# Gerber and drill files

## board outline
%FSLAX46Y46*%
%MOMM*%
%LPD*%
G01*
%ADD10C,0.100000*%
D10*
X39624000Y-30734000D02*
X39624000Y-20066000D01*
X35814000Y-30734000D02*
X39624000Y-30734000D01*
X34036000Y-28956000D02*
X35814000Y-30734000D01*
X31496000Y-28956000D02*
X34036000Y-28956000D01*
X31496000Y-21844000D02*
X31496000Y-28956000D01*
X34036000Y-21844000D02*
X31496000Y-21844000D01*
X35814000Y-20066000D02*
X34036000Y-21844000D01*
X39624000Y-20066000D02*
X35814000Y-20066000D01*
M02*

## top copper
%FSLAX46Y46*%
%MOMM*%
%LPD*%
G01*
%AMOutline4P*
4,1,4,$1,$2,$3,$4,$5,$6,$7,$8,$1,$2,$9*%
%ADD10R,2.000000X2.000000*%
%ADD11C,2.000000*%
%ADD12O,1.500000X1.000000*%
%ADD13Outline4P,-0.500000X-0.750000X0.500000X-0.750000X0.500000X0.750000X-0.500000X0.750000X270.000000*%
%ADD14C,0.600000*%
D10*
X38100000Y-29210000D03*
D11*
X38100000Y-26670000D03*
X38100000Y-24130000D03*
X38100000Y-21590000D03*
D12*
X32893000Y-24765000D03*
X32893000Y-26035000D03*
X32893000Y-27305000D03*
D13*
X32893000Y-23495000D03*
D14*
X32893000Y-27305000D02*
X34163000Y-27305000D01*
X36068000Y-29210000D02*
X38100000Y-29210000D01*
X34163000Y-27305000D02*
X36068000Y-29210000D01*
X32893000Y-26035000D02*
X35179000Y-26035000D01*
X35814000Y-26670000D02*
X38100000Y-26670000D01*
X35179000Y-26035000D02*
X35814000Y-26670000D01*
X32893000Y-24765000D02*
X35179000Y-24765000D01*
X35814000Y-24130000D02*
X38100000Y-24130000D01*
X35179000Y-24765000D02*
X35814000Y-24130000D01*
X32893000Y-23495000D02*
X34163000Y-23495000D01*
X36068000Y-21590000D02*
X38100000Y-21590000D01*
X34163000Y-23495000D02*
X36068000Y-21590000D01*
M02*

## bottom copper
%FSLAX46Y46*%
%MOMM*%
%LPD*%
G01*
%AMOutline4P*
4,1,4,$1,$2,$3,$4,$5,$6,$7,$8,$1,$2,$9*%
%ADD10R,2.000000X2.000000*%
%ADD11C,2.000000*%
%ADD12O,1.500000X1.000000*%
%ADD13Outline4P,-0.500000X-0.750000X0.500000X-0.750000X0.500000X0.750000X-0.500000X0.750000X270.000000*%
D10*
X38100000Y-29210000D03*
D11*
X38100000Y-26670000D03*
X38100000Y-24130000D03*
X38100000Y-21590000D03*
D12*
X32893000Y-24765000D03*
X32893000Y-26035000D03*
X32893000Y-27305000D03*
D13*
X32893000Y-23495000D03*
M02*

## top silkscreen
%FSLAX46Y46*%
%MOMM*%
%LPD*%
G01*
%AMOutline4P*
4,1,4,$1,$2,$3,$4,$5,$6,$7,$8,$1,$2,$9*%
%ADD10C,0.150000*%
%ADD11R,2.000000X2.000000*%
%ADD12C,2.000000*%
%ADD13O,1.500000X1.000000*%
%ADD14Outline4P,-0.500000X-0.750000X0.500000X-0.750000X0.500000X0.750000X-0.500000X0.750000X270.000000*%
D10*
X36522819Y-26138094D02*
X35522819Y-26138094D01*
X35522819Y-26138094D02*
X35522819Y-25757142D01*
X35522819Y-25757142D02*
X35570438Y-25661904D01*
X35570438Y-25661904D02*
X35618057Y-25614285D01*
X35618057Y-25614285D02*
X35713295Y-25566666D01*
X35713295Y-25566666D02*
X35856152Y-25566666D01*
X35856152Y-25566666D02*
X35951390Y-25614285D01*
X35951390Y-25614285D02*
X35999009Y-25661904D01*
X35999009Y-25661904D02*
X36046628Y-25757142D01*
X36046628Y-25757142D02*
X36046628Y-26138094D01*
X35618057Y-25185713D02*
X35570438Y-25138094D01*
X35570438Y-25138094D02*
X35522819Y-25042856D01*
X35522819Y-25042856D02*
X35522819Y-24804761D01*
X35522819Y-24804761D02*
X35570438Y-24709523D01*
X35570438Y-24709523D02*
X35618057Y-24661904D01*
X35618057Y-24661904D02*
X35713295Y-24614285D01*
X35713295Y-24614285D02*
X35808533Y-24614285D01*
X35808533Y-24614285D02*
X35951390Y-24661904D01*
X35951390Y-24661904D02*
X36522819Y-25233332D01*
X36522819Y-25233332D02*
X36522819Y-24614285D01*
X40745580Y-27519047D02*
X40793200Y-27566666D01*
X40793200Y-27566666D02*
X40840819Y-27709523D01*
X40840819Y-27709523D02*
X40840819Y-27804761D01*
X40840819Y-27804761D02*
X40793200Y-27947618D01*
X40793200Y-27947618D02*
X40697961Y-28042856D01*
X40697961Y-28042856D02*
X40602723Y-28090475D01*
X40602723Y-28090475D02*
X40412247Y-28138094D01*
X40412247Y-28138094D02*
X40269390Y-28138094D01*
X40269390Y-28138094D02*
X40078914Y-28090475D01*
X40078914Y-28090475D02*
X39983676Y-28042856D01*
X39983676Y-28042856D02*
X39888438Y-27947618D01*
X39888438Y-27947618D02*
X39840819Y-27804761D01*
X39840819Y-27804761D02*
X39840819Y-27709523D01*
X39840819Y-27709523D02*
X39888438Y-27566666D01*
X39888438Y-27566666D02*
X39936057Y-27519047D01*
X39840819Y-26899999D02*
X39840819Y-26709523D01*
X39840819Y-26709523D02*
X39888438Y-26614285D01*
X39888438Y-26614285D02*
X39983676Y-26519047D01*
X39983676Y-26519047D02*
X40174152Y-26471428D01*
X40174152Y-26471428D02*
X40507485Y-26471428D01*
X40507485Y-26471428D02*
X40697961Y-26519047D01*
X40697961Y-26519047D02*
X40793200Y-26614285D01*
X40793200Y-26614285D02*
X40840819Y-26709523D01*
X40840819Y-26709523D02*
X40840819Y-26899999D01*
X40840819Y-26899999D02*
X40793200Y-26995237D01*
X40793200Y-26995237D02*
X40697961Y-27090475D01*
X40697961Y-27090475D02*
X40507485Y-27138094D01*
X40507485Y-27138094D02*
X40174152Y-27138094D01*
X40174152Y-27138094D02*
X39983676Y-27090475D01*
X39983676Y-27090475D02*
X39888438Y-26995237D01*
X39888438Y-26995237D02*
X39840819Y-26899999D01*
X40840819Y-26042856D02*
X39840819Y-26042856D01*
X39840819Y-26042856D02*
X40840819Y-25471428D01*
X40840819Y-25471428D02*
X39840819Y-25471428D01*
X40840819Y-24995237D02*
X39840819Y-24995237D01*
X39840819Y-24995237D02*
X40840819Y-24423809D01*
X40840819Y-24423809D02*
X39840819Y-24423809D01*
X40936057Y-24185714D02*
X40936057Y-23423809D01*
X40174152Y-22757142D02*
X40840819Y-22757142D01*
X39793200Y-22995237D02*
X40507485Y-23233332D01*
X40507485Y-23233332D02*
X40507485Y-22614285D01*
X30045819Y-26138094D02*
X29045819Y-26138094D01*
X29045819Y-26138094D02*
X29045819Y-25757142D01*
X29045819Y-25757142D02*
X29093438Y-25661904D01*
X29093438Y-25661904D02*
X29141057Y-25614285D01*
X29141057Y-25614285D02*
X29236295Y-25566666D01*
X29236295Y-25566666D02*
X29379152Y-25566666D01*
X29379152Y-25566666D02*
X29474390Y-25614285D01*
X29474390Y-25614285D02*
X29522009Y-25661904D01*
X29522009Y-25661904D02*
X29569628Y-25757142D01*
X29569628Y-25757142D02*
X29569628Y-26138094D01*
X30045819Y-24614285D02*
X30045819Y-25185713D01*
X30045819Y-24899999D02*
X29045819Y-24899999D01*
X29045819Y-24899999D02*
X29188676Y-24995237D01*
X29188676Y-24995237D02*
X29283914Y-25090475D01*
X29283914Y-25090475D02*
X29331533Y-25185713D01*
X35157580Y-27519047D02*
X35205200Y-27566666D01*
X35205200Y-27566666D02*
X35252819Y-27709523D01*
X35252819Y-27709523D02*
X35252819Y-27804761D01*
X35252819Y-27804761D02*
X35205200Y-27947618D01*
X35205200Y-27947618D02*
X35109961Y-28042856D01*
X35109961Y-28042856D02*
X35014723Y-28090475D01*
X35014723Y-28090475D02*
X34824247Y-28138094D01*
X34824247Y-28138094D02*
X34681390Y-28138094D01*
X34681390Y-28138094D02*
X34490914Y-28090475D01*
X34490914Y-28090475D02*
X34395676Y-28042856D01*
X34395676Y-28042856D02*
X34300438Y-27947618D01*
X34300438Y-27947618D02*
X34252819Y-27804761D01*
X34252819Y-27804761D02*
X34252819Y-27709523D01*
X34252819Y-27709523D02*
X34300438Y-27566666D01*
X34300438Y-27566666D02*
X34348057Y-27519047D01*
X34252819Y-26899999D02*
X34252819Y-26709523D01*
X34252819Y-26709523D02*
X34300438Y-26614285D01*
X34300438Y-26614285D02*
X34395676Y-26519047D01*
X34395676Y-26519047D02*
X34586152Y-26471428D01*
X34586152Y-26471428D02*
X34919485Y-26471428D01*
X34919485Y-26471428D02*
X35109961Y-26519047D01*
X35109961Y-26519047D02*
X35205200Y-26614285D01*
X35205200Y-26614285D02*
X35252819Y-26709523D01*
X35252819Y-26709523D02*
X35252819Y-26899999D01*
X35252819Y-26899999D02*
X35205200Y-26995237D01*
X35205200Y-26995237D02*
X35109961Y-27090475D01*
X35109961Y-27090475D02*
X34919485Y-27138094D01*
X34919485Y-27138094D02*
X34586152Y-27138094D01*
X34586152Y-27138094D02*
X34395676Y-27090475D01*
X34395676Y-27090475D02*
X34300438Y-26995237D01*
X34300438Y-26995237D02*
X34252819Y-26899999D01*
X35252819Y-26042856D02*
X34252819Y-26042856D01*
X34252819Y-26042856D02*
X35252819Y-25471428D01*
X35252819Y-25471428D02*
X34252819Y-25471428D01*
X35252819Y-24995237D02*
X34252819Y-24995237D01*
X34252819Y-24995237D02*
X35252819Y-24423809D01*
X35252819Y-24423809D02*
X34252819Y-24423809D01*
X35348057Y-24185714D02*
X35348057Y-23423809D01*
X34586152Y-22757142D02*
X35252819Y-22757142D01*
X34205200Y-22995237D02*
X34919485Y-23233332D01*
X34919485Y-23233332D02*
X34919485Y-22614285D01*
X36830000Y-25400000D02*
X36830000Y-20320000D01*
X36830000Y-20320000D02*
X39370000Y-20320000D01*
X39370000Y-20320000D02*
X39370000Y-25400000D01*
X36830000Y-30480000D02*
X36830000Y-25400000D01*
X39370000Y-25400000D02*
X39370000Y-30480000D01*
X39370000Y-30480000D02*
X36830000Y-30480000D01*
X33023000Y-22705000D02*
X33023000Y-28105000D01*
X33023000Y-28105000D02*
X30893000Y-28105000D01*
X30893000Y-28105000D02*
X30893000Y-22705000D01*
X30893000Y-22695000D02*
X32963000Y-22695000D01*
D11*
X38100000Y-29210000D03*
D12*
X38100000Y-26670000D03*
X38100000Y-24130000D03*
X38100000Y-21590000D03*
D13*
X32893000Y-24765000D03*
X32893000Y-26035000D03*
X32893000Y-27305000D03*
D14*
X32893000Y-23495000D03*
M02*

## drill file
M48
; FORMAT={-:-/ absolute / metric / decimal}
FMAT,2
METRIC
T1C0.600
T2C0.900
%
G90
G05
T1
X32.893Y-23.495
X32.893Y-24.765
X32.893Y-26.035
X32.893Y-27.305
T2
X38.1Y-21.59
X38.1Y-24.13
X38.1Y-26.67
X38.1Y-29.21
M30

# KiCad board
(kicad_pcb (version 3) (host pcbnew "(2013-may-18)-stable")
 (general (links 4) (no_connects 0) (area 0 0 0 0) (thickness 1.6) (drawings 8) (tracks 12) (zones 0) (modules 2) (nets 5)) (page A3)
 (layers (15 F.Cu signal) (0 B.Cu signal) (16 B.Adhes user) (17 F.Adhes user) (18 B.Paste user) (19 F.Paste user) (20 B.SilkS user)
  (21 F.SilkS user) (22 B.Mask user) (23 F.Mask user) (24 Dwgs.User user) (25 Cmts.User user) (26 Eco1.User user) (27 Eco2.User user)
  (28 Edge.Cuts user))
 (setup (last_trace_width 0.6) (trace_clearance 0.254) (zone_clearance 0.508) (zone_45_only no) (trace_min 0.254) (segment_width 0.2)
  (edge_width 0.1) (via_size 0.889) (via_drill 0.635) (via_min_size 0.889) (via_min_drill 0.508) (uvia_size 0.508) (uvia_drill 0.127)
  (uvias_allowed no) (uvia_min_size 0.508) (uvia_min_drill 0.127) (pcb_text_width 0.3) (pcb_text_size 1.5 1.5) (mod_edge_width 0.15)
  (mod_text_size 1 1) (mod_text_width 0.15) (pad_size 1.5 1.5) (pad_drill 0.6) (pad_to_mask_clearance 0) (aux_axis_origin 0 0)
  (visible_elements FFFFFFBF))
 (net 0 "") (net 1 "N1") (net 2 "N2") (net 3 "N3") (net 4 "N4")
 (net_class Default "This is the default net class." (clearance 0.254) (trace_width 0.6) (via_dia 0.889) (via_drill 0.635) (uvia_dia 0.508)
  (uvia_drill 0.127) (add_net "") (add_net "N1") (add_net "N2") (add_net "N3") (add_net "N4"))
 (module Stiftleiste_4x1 (layer F.Cu) (at 38.1 25.4 90)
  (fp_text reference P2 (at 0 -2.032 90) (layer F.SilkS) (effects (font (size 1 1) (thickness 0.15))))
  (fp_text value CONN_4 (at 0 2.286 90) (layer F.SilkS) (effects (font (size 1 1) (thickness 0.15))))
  (fp_line (start 0 -1.27) (end 5.08 -1.27) (layer F.SilkS) (width 0.15))
  (fp_line (start 5.08 -1.27) (end 5.08 1.27) (layer F.SilkS) (width 0.15))
  (fp_line (start 5.08 1.27) (end 0 1.27) (layer F.SilkS) (width 0.15))
  (fp_line (start -5.08 -1.27) (end 0 -1.27) (layer F.SilkS) (width 0.15))
  (fp_line (start 0 1.27) (end -5.08 1.27) (layer F.SilkS) (width 0.15))
  (fp_line (start -5.08 1.27) (end -5.08 -1.27) (layer F.SilkS) (width 0.15))
  (pad 1 thru_hole rect (at -3.81 0 90) (size 2 2) (drill 0.9) (layers *.Cu *.Mask F.SilkS) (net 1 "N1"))
  (pad 2 thru_hole circle (at -1.27 0 90) (size 2 2) (drill 0.9) (layers *.Cu *.Mask F.SilkS) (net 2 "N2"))
  (pad 3 thru_hole circle (at 1.27 0 90) (size 2 2) (drill 0.9) (layers *.Cu *.Mask F.SilkS) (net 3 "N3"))
  (pad 4 thru_hole circle (at 3.81 0 90) (size 2 2) (drill 0.9) (layers *.Cu *.Mask F.SilkS) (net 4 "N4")))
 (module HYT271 (layer F.Cu) (at 33.02 25.4 270)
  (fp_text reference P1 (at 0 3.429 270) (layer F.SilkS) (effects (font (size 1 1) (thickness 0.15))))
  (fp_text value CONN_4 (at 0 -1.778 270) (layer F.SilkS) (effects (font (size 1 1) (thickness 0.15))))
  (fp_line (start -2.695 -0.003) (end 2.705 -0.003) (layer F.SilkS) (width 0.15))
  (fp_line (start 2.705 -0.003) (end 2.705 2.127) (layer F.SilkS) (width 0.15))
  (fp_line (start 2.705 2.127) (end -2.695 2.127) (layer F.SilkS) (width 0.15))
  (fp_line (start -2.705 2.127) (end -2.705 0.057) (layer F.SilkS) (width 0.15))
  (pad 2 thru_hole oval (at -0.635 0.127 270) (size 1 1.5) (drill 0.6) (layers *.Cu *.Mask F.SilkS) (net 3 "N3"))
  (pad 3 thru_hole oval (at 0.635 0.127 270) (size 1 1.5) (drill 0.6) (layers *.Cu *.Mask F.SilkS) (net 2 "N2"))
  (pad 4 thru_hole oval (at 1.905 0.127 270) (size 1 1.5) (drill 0.6) (layers *.Cu *.Mask F.SilkS) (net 1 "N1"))
  (pad 1 thru_hole trapezoid (at -1.905 0.127 270) (size 1 1.5) (drill 0.6) (layers *.Cu *.Mask F.SilkS) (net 4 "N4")))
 (gr_line (start 39.624 30.734) (end 39.624 20.066) (angle 90) (layer Edge.Cuts) (width 0.1))
 (gr_line (start 35.814 30.734) (end 39.624 30.734) (angle 90) (layer Edge.Cuts) (width 0.1))
 (gr_line (start 34.036 28.956) (end 35.814 30.734) (angle 90) (layer Edge.Cuts) (width 0.1))
 (gr_line (start 31.496 28.956) (end 34.036 28.956) (angle 90) (layer Edge.Cuts) (width 0.1))
 (gr_line (start 31.496 21.844) (end 31.496 28.956) (angle 90) (layer Edge.Cuts) (width 0.1))
 (gr_line (start 34.036 21.844) (end 31.496 21.844) (angle 90) (layer Edge.Cuts) (width 0.1))
 (gr_line (start 35.814 20.066) (end 34.036 21.844) (angle 90) (layer Edge.Cuts) (width 0.1))
 (gr_line (start 39.624 20.066) (end 35.814 20.066) (angle 90) (layer Edge.Cuts) (width 0.1))
 (segment (start 32.893 27.305) (end 34.163 27.305) (width 0.6) (layer F.Cu) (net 1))
 (segment (start 36.068 29.21) (end 38.1 29.21) (width 0.6) (layer F.Cu) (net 1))
 (segment (start 34.163 27.305) (end 36.068 29.21) (width 0.6) (layer F.Cu) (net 1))
 (segment (start 32.893 26.035) (end 35.179 26.035) (width 0.6) (layer F.Cu) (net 2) (status 400000))
 (segment (start 35.814 26.67) (end 38.1 26.67) (width 0.6) (layer F.Cu) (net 2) (status 800000))
 (segment (start 35.179 26.035) (end 35.814 26.67) (width 0.6) (layer F.Cu) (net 2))
 (segment (start 32.893 24.765) (end 35.179 24.765) (width 0.6) (layer F.Cu) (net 3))
 (segment (start 35.814 24.13) (end 38.1 24.13) (width 0.6) (layer F.Cu) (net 3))
 (segment (start 35.179 24.765) (end 35.814 24.13) (width 0.6) (layer F.Cu) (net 3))
 (segment (start 32.893 23.495) (end 34.163 23.495) (width 0.6) (layer F.Cu) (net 4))
 (segment (start 36.068 21.59) (end 38.1 21.59) (width 0.6) (layer F.Cu) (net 4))
 (segment (start 34.163 23.495) (end 36.068 21.59) (width 0.6) (layer F.Cu) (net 4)))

